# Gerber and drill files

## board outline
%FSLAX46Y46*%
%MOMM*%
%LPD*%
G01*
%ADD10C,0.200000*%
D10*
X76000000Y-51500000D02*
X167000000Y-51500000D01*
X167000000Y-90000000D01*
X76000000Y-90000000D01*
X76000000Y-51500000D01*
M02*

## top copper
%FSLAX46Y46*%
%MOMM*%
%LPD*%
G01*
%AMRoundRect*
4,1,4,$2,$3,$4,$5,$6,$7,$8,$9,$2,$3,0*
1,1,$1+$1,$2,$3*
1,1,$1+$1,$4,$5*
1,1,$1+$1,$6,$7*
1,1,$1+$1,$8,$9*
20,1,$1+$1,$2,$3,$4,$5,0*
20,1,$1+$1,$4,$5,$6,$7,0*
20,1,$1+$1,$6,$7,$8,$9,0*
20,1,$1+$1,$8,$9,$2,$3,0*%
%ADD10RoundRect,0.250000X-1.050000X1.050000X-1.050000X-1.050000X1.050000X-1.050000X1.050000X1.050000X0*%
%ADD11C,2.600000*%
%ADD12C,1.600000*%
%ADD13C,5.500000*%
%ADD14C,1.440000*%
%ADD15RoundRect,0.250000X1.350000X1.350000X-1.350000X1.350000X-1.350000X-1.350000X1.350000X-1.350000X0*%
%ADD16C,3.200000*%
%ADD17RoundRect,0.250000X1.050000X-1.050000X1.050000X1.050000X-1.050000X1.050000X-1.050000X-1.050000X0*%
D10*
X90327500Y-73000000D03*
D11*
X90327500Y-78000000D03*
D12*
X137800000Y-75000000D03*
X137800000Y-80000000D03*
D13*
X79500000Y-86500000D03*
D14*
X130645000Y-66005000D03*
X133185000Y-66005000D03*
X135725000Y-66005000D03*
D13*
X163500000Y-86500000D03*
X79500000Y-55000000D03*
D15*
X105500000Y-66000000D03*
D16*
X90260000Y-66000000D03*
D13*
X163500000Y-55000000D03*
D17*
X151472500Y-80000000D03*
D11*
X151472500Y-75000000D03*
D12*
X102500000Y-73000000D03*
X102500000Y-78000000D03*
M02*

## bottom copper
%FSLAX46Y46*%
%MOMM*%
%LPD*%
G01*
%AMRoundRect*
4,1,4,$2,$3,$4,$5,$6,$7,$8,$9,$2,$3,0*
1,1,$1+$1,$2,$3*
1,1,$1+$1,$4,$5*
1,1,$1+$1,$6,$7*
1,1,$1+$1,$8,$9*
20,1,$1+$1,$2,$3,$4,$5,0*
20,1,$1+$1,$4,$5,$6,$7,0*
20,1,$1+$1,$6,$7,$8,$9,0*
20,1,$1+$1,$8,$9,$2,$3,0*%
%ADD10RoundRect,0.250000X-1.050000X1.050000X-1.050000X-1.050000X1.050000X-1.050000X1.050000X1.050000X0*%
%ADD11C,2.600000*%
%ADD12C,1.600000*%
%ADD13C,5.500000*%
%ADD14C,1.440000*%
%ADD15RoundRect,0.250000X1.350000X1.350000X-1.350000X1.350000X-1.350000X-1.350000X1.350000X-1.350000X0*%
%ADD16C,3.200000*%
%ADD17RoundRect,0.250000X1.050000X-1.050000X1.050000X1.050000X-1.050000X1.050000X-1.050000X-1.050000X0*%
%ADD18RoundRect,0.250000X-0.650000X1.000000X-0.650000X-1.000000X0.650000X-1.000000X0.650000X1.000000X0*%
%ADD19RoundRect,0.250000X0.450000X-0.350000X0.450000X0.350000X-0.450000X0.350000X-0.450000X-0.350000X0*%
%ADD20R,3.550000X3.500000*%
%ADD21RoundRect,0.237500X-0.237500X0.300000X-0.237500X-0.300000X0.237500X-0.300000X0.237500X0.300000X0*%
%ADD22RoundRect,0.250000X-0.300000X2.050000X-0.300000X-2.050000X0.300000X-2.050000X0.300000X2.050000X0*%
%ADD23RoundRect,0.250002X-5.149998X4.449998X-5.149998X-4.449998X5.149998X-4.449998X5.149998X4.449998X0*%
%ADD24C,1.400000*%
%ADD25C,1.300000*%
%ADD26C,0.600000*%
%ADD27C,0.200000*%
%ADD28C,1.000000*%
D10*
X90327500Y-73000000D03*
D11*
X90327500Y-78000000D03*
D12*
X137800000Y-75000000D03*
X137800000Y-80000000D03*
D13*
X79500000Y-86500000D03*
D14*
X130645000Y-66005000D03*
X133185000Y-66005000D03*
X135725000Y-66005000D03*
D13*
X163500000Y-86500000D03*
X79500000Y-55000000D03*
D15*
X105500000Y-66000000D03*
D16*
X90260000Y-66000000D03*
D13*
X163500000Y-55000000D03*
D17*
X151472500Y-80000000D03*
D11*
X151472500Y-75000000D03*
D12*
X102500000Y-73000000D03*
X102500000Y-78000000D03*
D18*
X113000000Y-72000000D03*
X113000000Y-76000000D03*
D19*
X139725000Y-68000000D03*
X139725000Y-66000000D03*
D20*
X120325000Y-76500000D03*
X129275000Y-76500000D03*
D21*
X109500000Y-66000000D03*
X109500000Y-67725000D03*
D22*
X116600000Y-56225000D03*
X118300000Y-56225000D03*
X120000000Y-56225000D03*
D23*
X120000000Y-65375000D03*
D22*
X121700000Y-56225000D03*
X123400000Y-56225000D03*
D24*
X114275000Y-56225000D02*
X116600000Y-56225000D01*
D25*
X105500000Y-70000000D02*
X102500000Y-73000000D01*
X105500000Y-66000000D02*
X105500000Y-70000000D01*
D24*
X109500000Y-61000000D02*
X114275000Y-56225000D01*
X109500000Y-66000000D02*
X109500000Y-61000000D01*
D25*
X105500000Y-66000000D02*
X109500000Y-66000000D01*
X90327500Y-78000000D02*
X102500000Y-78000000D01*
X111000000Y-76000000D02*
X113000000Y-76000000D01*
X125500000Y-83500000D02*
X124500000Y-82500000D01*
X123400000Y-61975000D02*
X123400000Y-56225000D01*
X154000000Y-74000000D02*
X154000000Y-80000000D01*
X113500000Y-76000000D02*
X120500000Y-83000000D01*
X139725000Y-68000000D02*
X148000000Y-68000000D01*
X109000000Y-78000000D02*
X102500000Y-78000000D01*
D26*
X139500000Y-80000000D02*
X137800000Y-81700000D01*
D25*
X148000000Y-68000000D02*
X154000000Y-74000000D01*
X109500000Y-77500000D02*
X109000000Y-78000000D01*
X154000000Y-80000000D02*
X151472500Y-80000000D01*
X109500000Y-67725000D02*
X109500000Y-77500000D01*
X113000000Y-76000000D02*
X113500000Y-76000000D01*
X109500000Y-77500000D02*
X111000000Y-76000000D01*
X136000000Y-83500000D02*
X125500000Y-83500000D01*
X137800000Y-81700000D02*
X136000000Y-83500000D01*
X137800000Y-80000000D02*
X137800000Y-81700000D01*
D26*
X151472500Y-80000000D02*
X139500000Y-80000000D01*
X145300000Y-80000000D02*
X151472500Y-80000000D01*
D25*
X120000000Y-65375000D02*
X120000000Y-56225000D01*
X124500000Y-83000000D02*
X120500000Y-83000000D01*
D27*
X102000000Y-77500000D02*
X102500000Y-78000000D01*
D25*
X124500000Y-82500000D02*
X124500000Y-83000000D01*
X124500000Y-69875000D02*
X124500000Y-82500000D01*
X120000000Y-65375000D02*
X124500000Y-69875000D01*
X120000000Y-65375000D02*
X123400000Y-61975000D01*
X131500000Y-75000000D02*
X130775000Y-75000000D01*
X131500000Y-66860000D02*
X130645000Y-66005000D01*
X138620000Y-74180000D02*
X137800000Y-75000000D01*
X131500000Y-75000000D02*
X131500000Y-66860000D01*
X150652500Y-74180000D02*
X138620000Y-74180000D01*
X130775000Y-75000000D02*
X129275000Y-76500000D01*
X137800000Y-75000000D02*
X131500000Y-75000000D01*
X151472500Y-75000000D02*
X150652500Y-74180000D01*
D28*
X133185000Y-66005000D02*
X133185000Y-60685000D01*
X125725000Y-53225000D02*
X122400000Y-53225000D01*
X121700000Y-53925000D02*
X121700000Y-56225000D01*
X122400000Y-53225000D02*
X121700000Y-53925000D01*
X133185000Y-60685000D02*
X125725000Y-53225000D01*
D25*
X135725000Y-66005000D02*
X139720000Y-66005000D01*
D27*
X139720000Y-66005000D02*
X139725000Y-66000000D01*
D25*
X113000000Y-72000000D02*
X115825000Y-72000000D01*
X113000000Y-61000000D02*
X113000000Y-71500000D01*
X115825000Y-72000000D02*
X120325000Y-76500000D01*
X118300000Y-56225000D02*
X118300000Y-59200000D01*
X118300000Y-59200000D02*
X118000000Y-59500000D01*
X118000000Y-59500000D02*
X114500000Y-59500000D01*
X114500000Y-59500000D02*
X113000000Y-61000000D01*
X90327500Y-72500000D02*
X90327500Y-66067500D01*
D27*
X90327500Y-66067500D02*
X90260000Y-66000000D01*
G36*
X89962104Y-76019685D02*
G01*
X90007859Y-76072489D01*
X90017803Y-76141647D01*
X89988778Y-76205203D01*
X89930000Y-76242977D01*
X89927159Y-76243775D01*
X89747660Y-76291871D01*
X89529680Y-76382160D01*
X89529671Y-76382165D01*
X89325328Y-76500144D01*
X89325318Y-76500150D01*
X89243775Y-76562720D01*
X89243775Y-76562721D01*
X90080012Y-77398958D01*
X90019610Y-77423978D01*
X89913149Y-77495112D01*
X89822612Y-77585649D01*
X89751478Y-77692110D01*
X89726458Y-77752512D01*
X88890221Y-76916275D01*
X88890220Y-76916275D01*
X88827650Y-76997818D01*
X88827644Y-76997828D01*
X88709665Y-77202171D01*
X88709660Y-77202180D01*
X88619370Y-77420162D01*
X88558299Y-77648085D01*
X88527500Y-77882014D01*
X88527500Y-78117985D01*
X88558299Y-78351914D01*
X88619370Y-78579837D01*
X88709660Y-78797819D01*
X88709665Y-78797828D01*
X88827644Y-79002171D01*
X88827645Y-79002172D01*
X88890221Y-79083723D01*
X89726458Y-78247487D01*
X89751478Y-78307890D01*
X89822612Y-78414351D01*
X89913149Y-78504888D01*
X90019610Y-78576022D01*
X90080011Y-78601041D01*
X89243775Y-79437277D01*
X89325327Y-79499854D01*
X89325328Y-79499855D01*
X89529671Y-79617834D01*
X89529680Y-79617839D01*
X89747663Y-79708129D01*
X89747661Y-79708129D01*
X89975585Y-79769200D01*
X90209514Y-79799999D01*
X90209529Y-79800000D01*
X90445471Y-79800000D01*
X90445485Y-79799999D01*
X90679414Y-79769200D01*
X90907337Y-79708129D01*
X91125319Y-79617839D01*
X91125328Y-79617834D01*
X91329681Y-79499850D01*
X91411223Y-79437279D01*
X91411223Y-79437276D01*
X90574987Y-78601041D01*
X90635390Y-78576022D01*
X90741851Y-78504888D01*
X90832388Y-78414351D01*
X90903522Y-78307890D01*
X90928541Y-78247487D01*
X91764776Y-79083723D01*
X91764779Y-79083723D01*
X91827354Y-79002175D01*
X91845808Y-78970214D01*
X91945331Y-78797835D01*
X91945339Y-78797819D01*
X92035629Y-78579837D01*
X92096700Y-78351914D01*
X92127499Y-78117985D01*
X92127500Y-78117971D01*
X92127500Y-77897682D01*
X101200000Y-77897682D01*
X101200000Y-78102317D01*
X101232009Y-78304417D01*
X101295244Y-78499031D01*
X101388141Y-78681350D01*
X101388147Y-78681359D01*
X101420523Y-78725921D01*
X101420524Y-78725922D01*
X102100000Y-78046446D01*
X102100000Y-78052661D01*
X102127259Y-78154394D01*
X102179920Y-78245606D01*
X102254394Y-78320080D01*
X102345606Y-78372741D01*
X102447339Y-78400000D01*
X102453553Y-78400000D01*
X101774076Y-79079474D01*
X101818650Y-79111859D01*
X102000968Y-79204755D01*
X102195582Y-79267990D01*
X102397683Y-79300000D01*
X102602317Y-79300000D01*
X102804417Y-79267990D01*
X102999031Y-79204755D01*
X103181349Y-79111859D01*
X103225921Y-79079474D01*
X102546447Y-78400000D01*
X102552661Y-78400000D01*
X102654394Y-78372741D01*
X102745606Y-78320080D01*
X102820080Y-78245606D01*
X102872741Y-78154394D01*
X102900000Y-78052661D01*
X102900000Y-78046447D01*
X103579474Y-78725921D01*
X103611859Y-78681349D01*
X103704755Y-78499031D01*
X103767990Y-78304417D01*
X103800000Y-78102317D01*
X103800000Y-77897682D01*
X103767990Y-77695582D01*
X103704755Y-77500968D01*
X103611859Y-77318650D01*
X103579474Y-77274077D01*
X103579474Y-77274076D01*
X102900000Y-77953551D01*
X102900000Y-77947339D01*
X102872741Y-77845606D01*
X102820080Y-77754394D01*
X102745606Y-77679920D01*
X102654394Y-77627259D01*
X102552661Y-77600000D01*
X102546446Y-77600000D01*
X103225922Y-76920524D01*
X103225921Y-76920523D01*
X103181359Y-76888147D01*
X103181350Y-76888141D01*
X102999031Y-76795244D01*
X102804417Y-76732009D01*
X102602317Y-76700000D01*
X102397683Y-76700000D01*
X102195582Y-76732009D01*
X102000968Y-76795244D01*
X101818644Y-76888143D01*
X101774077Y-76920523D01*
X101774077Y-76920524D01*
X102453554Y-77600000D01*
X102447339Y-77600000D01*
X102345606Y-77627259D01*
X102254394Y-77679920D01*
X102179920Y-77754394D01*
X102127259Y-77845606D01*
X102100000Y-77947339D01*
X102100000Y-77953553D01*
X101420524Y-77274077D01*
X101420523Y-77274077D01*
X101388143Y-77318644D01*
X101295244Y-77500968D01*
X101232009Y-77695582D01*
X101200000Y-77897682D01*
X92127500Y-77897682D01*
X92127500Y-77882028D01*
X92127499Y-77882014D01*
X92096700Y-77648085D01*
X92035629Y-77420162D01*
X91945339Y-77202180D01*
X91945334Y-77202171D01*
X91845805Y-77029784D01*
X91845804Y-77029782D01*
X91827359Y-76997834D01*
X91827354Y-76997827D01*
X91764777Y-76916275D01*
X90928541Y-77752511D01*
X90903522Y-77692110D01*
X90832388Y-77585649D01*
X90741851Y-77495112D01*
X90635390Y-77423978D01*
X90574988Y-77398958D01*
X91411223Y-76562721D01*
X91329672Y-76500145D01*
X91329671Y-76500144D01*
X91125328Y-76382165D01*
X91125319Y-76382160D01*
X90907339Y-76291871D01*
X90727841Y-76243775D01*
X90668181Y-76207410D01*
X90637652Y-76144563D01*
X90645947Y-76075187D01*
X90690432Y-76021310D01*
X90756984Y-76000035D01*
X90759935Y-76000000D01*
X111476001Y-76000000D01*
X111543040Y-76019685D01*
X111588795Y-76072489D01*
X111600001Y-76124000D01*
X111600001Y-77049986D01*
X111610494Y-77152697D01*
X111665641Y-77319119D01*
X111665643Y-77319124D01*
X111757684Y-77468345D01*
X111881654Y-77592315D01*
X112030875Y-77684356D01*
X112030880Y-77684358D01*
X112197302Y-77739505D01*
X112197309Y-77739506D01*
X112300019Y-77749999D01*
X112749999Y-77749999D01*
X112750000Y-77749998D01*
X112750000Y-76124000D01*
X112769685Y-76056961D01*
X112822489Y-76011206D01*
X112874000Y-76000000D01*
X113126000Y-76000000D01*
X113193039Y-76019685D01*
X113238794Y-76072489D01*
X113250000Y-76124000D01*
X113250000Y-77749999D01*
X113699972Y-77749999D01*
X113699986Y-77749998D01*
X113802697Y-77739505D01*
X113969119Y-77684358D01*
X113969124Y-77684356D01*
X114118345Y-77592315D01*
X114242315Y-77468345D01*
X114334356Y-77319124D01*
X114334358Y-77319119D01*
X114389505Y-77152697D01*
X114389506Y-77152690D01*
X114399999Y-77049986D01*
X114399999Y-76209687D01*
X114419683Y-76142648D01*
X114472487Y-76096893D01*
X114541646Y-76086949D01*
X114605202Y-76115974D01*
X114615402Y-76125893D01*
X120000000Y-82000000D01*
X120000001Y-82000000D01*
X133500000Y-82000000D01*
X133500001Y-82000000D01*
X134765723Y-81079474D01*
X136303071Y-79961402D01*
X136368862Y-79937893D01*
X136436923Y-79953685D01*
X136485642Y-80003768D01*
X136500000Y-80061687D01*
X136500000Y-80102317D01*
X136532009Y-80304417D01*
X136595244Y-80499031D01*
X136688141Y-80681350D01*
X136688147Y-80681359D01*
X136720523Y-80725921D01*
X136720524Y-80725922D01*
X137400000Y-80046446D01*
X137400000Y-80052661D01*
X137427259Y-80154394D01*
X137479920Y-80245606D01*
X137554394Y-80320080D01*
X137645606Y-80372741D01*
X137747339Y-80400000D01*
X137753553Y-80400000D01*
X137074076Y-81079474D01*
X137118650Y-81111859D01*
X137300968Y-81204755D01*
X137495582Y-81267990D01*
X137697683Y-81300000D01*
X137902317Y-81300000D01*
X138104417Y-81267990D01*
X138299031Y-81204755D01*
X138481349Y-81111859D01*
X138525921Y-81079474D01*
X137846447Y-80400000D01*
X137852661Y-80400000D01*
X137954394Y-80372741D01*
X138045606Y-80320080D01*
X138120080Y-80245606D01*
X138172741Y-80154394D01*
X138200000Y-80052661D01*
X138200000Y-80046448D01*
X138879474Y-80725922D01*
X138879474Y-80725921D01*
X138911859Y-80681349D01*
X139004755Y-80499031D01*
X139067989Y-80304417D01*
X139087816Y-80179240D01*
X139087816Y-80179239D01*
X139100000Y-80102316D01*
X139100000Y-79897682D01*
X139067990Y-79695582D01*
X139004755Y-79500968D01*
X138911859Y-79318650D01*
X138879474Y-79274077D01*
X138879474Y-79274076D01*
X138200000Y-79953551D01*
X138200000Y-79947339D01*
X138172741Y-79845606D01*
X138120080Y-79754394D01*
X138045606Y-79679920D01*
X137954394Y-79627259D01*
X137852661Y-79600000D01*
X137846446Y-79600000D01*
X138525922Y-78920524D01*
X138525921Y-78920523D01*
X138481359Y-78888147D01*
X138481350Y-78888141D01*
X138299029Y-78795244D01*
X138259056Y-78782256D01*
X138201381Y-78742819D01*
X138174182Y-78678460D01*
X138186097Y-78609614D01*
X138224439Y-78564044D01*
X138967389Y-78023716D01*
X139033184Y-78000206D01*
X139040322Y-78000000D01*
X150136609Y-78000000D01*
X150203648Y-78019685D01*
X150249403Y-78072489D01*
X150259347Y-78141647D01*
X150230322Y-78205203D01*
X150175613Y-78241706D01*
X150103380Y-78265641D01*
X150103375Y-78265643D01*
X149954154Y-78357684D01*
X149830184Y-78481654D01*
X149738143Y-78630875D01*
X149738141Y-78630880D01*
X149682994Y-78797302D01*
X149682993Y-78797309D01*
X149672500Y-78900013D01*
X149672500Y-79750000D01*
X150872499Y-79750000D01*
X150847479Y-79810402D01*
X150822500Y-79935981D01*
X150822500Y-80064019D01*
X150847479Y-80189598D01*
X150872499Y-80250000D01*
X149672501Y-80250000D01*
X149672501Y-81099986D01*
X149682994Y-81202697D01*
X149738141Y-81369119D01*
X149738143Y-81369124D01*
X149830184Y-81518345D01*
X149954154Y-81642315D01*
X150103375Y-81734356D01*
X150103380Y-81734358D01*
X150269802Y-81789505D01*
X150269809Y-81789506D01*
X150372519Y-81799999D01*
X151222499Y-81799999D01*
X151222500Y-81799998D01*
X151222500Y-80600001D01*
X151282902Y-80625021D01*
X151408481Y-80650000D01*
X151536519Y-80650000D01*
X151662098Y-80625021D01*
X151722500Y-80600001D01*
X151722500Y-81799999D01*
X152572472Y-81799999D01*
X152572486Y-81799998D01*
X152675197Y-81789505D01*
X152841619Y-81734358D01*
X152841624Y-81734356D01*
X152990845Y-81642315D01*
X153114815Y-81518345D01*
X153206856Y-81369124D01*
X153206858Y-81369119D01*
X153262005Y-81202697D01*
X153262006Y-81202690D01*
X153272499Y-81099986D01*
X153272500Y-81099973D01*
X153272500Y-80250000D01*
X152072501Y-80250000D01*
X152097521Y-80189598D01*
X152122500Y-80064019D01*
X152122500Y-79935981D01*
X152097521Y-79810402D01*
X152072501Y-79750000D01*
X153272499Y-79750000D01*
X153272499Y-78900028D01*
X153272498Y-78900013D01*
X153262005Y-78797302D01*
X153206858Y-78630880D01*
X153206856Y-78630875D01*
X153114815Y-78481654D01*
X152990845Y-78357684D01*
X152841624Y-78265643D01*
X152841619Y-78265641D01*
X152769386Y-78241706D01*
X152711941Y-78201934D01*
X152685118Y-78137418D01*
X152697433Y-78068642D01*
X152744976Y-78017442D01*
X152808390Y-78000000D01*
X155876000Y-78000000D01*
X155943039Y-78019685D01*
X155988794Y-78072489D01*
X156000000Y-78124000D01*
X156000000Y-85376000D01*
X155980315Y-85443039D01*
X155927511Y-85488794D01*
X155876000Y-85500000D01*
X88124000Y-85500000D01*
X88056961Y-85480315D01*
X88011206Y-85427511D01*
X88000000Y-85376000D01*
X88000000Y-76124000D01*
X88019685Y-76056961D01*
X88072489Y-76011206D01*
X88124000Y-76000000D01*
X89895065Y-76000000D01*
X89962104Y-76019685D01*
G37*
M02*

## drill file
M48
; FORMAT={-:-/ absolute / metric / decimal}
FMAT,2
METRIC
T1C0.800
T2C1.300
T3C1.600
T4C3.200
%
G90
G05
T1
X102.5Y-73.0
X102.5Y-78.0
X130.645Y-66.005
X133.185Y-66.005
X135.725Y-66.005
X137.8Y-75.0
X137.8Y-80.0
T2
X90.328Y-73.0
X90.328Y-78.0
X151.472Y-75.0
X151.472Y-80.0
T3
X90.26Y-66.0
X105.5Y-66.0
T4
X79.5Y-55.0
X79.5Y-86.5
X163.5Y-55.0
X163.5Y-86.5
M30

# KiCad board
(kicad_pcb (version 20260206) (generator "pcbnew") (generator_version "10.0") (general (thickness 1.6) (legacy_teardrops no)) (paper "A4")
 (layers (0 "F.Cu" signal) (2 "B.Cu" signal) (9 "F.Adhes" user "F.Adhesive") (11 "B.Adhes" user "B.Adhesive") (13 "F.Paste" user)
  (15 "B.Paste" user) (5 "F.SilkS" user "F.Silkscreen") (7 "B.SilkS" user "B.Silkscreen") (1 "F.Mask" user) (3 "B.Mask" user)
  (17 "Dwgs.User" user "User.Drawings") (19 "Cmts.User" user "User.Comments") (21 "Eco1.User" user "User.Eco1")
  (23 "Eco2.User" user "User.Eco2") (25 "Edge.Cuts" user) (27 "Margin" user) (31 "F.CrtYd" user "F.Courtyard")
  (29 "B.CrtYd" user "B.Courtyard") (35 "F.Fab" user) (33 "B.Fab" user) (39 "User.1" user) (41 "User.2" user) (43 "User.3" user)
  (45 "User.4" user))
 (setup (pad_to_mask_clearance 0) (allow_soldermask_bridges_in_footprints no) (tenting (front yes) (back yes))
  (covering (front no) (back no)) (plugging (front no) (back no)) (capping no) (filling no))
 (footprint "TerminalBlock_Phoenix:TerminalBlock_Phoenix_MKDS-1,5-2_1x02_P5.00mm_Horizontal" (layer "F.Cu") (at 90.3275 73 -90)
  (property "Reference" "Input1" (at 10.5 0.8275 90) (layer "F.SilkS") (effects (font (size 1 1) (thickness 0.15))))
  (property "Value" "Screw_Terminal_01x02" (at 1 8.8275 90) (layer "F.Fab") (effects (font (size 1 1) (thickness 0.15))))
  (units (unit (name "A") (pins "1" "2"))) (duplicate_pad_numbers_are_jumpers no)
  (pad "1" thru_hole roundrect (at 0 0 270) (size 2.6 2.6) (drill 1.3) (layers "*.Cu" "*.Mask") (remove_unused_layers no)
   (roundrect_rratio 0.096154) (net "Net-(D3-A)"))
  (pad "2" thru_hole circle (at 5 0 270) (size 2.6 2.6) (drill 1.3) (layers "*.Cu" "*.Mask") (remove_unused_layers no) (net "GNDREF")))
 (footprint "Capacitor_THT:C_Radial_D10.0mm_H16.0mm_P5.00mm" (layer "F.Cu") (at 137.8 75 -90)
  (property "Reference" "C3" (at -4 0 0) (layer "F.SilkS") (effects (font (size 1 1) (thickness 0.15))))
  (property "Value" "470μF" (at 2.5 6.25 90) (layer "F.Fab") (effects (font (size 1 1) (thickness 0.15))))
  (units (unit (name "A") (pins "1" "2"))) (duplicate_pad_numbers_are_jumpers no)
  (pad "1" thru_hole circle (at 0 0 270) (size 1.6 1.6) (drill 0.8) (layers "*.Cu" "*.Mask") (remove_unused_layers no)
   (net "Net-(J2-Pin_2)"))
  (pad "2" thru_hole circle (at 5 0 270) (size 1.6 1.6) (drill 0.8) (layers "*.Cu" "*.Mask") (remove_unused_layers no) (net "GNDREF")))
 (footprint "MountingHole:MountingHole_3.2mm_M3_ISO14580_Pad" (layer "F.Cu") (at 79.5 86.5)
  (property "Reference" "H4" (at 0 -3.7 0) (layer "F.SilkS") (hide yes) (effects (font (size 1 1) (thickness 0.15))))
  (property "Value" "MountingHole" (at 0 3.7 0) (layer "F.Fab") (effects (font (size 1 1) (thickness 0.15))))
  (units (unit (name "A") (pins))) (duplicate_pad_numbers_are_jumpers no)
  (pad "1" thru_hole circle (at 0 0) (size 5.5 5.5) (drill 3.2) (layers "*.Cu" "*.Mask") (remove_unused_layers no) (zone_connect 2)))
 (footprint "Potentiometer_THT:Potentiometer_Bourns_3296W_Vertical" (layer "F.Cu") (at 130.645 66.005 180)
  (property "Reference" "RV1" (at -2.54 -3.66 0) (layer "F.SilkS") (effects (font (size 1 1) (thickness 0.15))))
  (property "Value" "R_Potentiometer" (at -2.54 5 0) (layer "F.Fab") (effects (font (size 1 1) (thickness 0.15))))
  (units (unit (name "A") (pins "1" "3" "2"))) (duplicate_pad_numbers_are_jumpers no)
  (pad "1" thru_hole circle (at 0 0 180) (size 1.44 1.44) (drill 0.8) (layers "*.Cu" "*.Mask") (remove_unused_layers no)
   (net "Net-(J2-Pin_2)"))
  (pad "2" thru_hole circle (at -2.54 0 180) (size 1.44 1.44) (drill 0.8) (layers "*.Cu" "*.Mask") (remove_unused_layers no)
   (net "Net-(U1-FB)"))
  (pad "3" thru_hole circle (at -5.08 0 180) (size 1.44 1.44) (drill 0.8) (layers "*.Cu" "*.Mask") (remove_unused_layers no)
   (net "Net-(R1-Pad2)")))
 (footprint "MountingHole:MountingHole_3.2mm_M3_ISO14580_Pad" (layer "F.Cu") (at 163.5 86.5)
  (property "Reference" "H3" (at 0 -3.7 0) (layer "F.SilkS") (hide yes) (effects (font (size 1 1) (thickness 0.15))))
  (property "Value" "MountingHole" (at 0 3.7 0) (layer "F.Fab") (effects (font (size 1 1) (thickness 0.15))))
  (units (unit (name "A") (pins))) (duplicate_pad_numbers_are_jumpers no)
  (pad "1" thru_hole circle (at 0 0) (size 5.5 5.5) (drill 3.2) (layers "*.Cu" "*.Mask") (remove_unused_layers no) (zone_connect 2)))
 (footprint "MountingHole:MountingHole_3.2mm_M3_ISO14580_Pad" (layer "F.Cu") (at 79.5 55)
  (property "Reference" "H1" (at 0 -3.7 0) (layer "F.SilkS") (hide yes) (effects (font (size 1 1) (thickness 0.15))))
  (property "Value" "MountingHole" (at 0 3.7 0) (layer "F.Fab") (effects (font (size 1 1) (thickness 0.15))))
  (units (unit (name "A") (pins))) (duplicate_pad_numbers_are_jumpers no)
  (pad "1" thru_hole circle (at 0 0) (size 5.5 5.5) (drill 3.2) (layers "*.Cu" "*.Mask") (remove_unused_layers no) (zone_connect 2)))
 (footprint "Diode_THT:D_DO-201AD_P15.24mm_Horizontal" (layer "F.Cu") (at 105.5 66 180)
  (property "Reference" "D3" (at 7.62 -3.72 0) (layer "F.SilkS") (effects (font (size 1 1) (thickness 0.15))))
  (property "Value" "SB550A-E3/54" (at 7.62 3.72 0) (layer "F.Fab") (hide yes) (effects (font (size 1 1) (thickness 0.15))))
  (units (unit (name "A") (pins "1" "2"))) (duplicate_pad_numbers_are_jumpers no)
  (pad "1" thru_hole roundrect (at 0 0 180) (size 3.2 3.2) (drill 1.6) (layers "*.Cu" "*.Mask") (remove_unused_layers no)
   (roundrect_rratio 0.078125) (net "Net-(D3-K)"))
  (pad "2" thru_hole circle (at 15.24 0 180) (size 3.2 3.2) (drill 1.6) (layers "*.Cu" "*.Mask") (remove_unused_layers no)
   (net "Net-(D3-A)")))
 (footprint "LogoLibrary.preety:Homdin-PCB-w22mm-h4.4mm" (layer "F.Cu") (at 143 55)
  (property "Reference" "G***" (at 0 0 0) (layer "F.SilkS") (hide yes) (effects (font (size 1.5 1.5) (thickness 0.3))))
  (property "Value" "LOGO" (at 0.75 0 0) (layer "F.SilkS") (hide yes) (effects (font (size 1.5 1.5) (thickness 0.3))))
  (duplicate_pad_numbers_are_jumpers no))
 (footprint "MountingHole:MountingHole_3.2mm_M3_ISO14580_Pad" (layer "F.Cu") (at 163.5 55)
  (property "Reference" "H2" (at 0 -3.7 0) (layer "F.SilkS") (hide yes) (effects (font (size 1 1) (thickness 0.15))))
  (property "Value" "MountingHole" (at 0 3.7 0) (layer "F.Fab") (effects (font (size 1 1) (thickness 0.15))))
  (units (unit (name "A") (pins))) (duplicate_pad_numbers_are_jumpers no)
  (pad "1" thru_hole circle (at 0 0) (size 5.5 5.5) (drill 3.2) (layers "*.Cu" "*.Mask") (remove_unused_layers no) (zone_connect 2)))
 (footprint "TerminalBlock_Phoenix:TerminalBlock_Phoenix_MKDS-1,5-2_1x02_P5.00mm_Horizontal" (layer "F.Cu") (at 151.4725 80 90)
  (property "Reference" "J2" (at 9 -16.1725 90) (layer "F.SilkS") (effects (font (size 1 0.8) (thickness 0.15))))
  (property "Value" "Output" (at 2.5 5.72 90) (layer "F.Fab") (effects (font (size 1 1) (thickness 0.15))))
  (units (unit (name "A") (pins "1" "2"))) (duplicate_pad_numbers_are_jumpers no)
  (pad "1" thru_hole roundrect (at 0 0 90) (size 2.6 2.6) (drill 1.3) (layers "*.Cu" "*.Mask") (remove_unused_layers no)
   (roundrect_rratio 0.096154) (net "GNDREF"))
  (pad "2" thru_hole circle (at 5 0 90) (size 2.6 2.6) (drill 1.3) (layers "*.Cu" "*.Mask") (remove_unused_layers no) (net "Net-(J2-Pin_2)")))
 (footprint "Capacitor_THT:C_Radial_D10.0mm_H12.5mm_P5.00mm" (layer "F.Cu") (at 102.5 73 -90)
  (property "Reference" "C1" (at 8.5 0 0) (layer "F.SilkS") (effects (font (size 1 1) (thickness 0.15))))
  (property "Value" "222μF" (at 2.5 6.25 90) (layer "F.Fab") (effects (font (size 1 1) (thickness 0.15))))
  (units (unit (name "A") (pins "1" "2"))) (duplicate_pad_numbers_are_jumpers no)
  (pad "1" thru_hole circle (at 0 0 270) (size 1.6 1.6) (drill 0.8) (layers "*.Cu" "*.Mask") (remove_unused_layers no) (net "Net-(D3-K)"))
  (pad "2" thru_hole circle (at 5 0 270) (size 1.6 1.6) (drill 0.8) (layers "*.Cu" "*.Mask") (remove_unused_layers no) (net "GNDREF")))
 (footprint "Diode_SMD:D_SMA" (layer "B.Cu") (at 113 74 -90)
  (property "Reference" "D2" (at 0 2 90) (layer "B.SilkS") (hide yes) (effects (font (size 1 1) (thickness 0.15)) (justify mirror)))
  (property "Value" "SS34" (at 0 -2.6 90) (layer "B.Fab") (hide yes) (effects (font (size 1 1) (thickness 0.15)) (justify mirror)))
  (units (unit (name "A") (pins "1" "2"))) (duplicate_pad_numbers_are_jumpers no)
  (pad "1" smd roundrect (at -2 0 270) (size 2.5 1.8) (layers "B.Cu" "B.Mask" "B.Paste") (roundrect_rratio 0.1388888889) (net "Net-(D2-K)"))
  (pad "2" smd roundrect (at 2 0 270) (size 2.5 1.8) (layers "B.Cu" "B.Mask" "B.Paste") (roundrect_rratio 0.1388888889) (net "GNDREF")))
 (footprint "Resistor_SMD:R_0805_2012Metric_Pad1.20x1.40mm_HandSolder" (layer "B.Cu") (at 139.725 67 90)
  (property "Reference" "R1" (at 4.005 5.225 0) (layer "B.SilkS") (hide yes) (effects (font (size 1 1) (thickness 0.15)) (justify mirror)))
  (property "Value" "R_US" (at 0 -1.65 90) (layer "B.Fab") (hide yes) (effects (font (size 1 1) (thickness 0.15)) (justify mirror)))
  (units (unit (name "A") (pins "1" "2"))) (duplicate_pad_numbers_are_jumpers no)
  (pad "1" smd roundrect (at -1 0 90) (size 1.2 1.4) (layers "B.Cu" "B.Mask" "B.Paste") (roundrect_rratio 0.208333) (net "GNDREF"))
  (pad "2" smd roundrect (at 1 0 90) (size 1.2 1.4) (layers "B.Cu" "B.Mask" "B.Paste") (roundrect_rratio 0.208333) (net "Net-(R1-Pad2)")))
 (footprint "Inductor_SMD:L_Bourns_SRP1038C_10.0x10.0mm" (layer "B.Cu") (at 124.8 76.5)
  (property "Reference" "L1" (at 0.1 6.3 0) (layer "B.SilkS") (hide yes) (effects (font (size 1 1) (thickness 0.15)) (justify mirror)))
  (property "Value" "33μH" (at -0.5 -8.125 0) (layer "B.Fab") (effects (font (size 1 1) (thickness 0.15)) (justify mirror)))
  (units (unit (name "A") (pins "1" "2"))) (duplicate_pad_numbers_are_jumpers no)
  (pad "1" smd rect (at -4.475 0) (size 3.55 3.5) (layers "B.Cu" "B.Mask" "B.Paste") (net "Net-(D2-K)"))
  (pad "2" smd rect (at 4.475 0) (size 3.55 3.5) (layers "B.Cu" "B.Mask" "B.Paste") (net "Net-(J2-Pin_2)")))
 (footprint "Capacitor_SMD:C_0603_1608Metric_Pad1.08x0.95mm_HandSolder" (layer "B.Cu") (at 109.5 66.8625 -90)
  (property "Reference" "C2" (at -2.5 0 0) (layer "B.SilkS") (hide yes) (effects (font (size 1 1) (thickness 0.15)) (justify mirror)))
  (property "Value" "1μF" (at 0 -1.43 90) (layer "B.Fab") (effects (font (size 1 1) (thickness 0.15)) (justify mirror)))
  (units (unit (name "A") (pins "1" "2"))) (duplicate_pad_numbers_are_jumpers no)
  (pad "1" smd roundrect (at -0.8625 0 270) (size 1.075 0.95) (layers "B.Cu" "B.Mask" "B.Paste") (roundrect_rratio 0.25) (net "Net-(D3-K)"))
  (pad "2" smd roundrect (at 0.8625 0 270) (size 1.075 0.95) (layers "B.Cu" "B.Mask" "B.Paste") (roundrect_rratio 0.25) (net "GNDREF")))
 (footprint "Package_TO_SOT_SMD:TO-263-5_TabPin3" (layer "B.Cu") (at 120 63.875 -90)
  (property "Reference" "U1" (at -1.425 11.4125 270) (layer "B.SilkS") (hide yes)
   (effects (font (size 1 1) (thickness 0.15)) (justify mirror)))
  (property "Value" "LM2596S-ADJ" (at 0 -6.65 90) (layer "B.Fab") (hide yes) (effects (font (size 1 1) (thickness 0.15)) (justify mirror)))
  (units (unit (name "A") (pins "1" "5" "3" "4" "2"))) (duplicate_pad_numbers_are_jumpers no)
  (pad "" smd roundrect (at -0.925 -2.775 270) (size 4.55 5.25) (layers "B.Paste") (roundrect_rratio 0.054945))
  (pad "" smd roundrect (at -0.925 2.775 270) (size 4.55 5.25) (layers "B.Paste") (roundrect_rratio 0.054945))
  (pad "" smd roundrect (at 3.925 -2.775 270) (size 4.55 5.25) (layers "B.Paste") (roundrect_rratio 0.054945))
  (pad "" smd roundrect (at 3.925 2.775 270) (size 4.55 5.25) (layers "B.Paste") (roundrect_rratio 0.054945))
  (pad "1" smd roundrect (at -7.65 3.4 270) (size 4.6 1.1) (layers "B.Cu" "B.Mask" "B.Paste") (roundrect_rratio 0.227273) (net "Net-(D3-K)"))
  (pad "2" smd roundrect (at -7.65 1.7 270) (size 4.6 1.1) (layers "B.Cu" "B.Mask" "B.Paste") (roundrect_rratio 0.227273) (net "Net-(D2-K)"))
  (pad "3" smd roundrect (at -7.65 0 270) (size 4.6 1.1) (layers "B.Cu" "B.Mask" "B.Paste") (roundrect_rratio 0.227273) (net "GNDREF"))
  (pad "3" smd roundrect (at 1.5 0 270) (size 9.4 10.8) (layers "B.Cu" "B.Mask") (roundrect_rratio 0.026596) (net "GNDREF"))
  (pad "4" smd roundrect (at -7.65 -1.7 270) (size 4.6 1.1) (layers "B.Cu" "B.Mask" "B.Paste") (roundrect_rratio 0.227273)
   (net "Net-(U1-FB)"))
  (pad "5" smd roundrect (at -7.65 -3.4 270) (size 4.6 1.1) (layers "B.Cu" "B.Mask" "B.Paste") (roundrect_rratio 0.227273) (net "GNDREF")))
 (gr_rect (start 76 51.5) (end 167 90) (stroke (width 0.2) (type solid)) (fill no) (layer "Edge.Cuts"))
 (segment (start 114.275 56.225) (end 116.6 56.225) (width 1.4) (layer "B.Cu") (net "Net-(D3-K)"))
 (segment (start 105.5 70) (end 102.5 73) (width 1.3) (layer "B.Cu") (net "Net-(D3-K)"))
 (segment (start 105.5 66) (end 105.5 70) (width 1.3) (layer "B.Cu") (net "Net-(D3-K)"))
 (segment (start 109.5 61) (end 114.275 56.225) (width 1.4) (layer "B.Cu") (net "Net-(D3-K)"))
 (segment (start 109.5 66) (end 109.5 61) (width 1.4) (layer "B.Cu") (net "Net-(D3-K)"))
 (segment (start 105.5 66) (end 109.5 66) (width 1.3) (layer "B.Cu") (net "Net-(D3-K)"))
 (segment (start 90.3275 78) (end 102.5 78) (width 1.3) (layer "B.Cu") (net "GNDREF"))
 (segment (start 111 76) (end 113 76) (width 1.3) (layer "B.Cu") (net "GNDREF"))
 (segment (start 125.5 83.5) (end 124.5 82.5) (width 1.3) (layer "B.Cu") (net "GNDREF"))
 (segment (start 123.4 61.975) (end 123.4 56.225) (width 1.3) (layer "B.Cu") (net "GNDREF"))
 (segment (start 154 74) (end 154 80) (width 1.3) (layer "B.Cu") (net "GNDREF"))
 (segment (start 113.5 76) (end 120.5 83) (width 1.3) (layer "B.Cu") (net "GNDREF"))
 (segment (start 139.725 68) (end 148 68) (width 1.3) (layer "B.Cu") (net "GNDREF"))
 (segment (start 109 78) (end 102.5 78) (width 1.3) (layer "B.Cu") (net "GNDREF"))
 (segment (start 139.5 80) (end 137.8 81.7) (width 0.6) (layer "B.Cu") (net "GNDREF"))
 (segment (start 148 68) (end 154 74) (width 1.3) (layer "B.Cu") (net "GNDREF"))
 (segment (start 109.5 77.5) (end 109 78) (width 1.3) (layer "B.Cu") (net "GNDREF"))
 (segment (start 154 80) (end 151.4725 80) (width 1.3) (layer "B.Cu") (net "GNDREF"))
 (segment (start 109.5 67.725) (end 109.5 77.5) (width 1.3) (layer "B.Cu") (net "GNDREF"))
 (segment (start 113 76) (end 113.5 76) (width 1.3) (layer "B.Cu") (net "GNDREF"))
 (segment (start 109.5 77.5) (end 111 76) (width 1.3) (layer "B.Cu") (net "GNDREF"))
 (segment (start 136 83.5) (end 125.5 83.5) (width 1.3) (layer "B.Cu") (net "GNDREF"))
 (segment (start 137.8 81.7) (end 136 83.5) (width 1.3) (layer "B.Cu") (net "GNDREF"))
 (segment (start 137.8 80) (end 137.8 81.7) (width 1.3) (layer "B.Cu") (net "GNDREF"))
 (segment (start 151.4725 80) (end 139.5 80) (width 0.6) (layer "B.Cu") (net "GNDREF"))
 (segment (start 145.3 80) (end 151.4725 80) (width 0.6) (layer "B.Cu") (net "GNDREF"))
 (segment (start 120 65.375) (end 120 56.225) (width 1.3) (layer "B.Cu") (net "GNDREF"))
 (segment (start 124.5 83) (end 120.5 83) (width 1.3) (layer "B.Cu") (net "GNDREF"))
 (segment (start 102 77.5) (end 102.5 78) (width 0.2) (layer "B.Cu") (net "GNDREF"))
 (segment (start 124.5 82.5) (end 124.5 83) (width 1.3) (layer "B.Cu") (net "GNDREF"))
 (segment (start 124.5 69.875) (end 124.5 82.5) (width 1.3) (layer "B.Cu") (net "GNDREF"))
 (segment (start 120 65.375) (end 124.5 69.875) (width 1.3) (layer "B.Cu") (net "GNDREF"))
 (segment (start 120 65.375) (end 123.4 61.975) (width 1.3) (layer "B.Cu") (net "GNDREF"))
 (segment (start 131.5 75) (end 130.775 75) (width 1.3) (layer "B.Cu") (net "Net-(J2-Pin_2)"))
 (segment (start 131.5 66.86) (end 130.645 66.005) (width 1.3) (layer "B.Cu") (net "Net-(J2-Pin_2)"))
 (segment (start 138.62 74.18) (end 137.8 75) (width 1.3) (layer "B.Cu") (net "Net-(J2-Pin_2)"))
 (segment (start 131.5 75) (end 131.5 66.86) (width 1.3) (layer "B.Cu") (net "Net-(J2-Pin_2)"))
 (segment (start 150.6525 74.18) (end 138.62 74.18) (width 1.3) (layer "B.Cu") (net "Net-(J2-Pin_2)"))
 (segment (start 130.775 75) (end 129.275 76.5) (width 1.3) (layer "B.Cu") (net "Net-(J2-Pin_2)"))
 (segment (start 137.8 75) (end 131.5 75) (width 1.3) (layer "B.Cu") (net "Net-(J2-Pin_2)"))
 (segment (start 151.4725 75) (end 150.6525 74.18) (width 1.3) (layer "B.Cu") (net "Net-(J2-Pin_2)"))
 (segment (start 133.185 66.005) (end 133.185 60.685) (width 1) (layer "B.Cu") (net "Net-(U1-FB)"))
 (segment (start 125.725 53.225) (end 122.4 53.225) (width 1) (layer "B.Cu") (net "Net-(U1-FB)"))
 (segment (start 121.7 53.925) (end 121.7 56.225) (width 1) (layer "B.Cu") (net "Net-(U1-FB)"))
 (segment (start 122.4 53.225) (end 121.7 53.925) (width 1) (layer "B.Cu") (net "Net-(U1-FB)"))
 (segment (start 133.185 60.685) (end 125.725 53.225) (width 1) (layer "B.Cu") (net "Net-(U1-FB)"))
 (segment (start 135.725 66.005) (end 139.72 66.005) (width 1.3) (layer "B.Cu") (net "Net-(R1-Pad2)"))
 (segment (start 139.72 66.005) (end 139.725 66) (width 0.2) (layer "B.Cu") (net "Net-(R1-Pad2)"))
 (segment (start 113 72) (end 115.825 72) (width 1.3) (layer "B.Cu") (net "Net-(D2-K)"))
 (segment (start 113 61) (end 113 71.5) (width 1.3) (layer "B.Cu") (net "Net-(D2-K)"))
 (segment (start 115.825 72) (end 120.325 76.5) (width 1.3) (layer "B.Cu") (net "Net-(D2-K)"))
 (segment (start 118.3 56.225) (end 118.3 59.2) (width 1.3) (layer "B.Cu") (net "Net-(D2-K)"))
 (segment (start 118.3 59.2) (end 118 59.5) (width 1.3) (layer "B.Cu") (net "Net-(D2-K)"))
 (segment (start 118 59.5) (end 114.5 59.5) (width 1.3) (layer "B.Cu") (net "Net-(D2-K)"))
 (segment (start 114.5 59.5) (end 113 61) (width 1.3) (layer "B.Cu") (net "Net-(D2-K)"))
 (segment (start 90.3275 72.5) (end 90.3275 66.0675) (width 1.3) (layer "B.Cu") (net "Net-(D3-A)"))
 (segment (start 90.3275 66.0675) (end 90.26 66) (width 0.2) (layer "B.Cu") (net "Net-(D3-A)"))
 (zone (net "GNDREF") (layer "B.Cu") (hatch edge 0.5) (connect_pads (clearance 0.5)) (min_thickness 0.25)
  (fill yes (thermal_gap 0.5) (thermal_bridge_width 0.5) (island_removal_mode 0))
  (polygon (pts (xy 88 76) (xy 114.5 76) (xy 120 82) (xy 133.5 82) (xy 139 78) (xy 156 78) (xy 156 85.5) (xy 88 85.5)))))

